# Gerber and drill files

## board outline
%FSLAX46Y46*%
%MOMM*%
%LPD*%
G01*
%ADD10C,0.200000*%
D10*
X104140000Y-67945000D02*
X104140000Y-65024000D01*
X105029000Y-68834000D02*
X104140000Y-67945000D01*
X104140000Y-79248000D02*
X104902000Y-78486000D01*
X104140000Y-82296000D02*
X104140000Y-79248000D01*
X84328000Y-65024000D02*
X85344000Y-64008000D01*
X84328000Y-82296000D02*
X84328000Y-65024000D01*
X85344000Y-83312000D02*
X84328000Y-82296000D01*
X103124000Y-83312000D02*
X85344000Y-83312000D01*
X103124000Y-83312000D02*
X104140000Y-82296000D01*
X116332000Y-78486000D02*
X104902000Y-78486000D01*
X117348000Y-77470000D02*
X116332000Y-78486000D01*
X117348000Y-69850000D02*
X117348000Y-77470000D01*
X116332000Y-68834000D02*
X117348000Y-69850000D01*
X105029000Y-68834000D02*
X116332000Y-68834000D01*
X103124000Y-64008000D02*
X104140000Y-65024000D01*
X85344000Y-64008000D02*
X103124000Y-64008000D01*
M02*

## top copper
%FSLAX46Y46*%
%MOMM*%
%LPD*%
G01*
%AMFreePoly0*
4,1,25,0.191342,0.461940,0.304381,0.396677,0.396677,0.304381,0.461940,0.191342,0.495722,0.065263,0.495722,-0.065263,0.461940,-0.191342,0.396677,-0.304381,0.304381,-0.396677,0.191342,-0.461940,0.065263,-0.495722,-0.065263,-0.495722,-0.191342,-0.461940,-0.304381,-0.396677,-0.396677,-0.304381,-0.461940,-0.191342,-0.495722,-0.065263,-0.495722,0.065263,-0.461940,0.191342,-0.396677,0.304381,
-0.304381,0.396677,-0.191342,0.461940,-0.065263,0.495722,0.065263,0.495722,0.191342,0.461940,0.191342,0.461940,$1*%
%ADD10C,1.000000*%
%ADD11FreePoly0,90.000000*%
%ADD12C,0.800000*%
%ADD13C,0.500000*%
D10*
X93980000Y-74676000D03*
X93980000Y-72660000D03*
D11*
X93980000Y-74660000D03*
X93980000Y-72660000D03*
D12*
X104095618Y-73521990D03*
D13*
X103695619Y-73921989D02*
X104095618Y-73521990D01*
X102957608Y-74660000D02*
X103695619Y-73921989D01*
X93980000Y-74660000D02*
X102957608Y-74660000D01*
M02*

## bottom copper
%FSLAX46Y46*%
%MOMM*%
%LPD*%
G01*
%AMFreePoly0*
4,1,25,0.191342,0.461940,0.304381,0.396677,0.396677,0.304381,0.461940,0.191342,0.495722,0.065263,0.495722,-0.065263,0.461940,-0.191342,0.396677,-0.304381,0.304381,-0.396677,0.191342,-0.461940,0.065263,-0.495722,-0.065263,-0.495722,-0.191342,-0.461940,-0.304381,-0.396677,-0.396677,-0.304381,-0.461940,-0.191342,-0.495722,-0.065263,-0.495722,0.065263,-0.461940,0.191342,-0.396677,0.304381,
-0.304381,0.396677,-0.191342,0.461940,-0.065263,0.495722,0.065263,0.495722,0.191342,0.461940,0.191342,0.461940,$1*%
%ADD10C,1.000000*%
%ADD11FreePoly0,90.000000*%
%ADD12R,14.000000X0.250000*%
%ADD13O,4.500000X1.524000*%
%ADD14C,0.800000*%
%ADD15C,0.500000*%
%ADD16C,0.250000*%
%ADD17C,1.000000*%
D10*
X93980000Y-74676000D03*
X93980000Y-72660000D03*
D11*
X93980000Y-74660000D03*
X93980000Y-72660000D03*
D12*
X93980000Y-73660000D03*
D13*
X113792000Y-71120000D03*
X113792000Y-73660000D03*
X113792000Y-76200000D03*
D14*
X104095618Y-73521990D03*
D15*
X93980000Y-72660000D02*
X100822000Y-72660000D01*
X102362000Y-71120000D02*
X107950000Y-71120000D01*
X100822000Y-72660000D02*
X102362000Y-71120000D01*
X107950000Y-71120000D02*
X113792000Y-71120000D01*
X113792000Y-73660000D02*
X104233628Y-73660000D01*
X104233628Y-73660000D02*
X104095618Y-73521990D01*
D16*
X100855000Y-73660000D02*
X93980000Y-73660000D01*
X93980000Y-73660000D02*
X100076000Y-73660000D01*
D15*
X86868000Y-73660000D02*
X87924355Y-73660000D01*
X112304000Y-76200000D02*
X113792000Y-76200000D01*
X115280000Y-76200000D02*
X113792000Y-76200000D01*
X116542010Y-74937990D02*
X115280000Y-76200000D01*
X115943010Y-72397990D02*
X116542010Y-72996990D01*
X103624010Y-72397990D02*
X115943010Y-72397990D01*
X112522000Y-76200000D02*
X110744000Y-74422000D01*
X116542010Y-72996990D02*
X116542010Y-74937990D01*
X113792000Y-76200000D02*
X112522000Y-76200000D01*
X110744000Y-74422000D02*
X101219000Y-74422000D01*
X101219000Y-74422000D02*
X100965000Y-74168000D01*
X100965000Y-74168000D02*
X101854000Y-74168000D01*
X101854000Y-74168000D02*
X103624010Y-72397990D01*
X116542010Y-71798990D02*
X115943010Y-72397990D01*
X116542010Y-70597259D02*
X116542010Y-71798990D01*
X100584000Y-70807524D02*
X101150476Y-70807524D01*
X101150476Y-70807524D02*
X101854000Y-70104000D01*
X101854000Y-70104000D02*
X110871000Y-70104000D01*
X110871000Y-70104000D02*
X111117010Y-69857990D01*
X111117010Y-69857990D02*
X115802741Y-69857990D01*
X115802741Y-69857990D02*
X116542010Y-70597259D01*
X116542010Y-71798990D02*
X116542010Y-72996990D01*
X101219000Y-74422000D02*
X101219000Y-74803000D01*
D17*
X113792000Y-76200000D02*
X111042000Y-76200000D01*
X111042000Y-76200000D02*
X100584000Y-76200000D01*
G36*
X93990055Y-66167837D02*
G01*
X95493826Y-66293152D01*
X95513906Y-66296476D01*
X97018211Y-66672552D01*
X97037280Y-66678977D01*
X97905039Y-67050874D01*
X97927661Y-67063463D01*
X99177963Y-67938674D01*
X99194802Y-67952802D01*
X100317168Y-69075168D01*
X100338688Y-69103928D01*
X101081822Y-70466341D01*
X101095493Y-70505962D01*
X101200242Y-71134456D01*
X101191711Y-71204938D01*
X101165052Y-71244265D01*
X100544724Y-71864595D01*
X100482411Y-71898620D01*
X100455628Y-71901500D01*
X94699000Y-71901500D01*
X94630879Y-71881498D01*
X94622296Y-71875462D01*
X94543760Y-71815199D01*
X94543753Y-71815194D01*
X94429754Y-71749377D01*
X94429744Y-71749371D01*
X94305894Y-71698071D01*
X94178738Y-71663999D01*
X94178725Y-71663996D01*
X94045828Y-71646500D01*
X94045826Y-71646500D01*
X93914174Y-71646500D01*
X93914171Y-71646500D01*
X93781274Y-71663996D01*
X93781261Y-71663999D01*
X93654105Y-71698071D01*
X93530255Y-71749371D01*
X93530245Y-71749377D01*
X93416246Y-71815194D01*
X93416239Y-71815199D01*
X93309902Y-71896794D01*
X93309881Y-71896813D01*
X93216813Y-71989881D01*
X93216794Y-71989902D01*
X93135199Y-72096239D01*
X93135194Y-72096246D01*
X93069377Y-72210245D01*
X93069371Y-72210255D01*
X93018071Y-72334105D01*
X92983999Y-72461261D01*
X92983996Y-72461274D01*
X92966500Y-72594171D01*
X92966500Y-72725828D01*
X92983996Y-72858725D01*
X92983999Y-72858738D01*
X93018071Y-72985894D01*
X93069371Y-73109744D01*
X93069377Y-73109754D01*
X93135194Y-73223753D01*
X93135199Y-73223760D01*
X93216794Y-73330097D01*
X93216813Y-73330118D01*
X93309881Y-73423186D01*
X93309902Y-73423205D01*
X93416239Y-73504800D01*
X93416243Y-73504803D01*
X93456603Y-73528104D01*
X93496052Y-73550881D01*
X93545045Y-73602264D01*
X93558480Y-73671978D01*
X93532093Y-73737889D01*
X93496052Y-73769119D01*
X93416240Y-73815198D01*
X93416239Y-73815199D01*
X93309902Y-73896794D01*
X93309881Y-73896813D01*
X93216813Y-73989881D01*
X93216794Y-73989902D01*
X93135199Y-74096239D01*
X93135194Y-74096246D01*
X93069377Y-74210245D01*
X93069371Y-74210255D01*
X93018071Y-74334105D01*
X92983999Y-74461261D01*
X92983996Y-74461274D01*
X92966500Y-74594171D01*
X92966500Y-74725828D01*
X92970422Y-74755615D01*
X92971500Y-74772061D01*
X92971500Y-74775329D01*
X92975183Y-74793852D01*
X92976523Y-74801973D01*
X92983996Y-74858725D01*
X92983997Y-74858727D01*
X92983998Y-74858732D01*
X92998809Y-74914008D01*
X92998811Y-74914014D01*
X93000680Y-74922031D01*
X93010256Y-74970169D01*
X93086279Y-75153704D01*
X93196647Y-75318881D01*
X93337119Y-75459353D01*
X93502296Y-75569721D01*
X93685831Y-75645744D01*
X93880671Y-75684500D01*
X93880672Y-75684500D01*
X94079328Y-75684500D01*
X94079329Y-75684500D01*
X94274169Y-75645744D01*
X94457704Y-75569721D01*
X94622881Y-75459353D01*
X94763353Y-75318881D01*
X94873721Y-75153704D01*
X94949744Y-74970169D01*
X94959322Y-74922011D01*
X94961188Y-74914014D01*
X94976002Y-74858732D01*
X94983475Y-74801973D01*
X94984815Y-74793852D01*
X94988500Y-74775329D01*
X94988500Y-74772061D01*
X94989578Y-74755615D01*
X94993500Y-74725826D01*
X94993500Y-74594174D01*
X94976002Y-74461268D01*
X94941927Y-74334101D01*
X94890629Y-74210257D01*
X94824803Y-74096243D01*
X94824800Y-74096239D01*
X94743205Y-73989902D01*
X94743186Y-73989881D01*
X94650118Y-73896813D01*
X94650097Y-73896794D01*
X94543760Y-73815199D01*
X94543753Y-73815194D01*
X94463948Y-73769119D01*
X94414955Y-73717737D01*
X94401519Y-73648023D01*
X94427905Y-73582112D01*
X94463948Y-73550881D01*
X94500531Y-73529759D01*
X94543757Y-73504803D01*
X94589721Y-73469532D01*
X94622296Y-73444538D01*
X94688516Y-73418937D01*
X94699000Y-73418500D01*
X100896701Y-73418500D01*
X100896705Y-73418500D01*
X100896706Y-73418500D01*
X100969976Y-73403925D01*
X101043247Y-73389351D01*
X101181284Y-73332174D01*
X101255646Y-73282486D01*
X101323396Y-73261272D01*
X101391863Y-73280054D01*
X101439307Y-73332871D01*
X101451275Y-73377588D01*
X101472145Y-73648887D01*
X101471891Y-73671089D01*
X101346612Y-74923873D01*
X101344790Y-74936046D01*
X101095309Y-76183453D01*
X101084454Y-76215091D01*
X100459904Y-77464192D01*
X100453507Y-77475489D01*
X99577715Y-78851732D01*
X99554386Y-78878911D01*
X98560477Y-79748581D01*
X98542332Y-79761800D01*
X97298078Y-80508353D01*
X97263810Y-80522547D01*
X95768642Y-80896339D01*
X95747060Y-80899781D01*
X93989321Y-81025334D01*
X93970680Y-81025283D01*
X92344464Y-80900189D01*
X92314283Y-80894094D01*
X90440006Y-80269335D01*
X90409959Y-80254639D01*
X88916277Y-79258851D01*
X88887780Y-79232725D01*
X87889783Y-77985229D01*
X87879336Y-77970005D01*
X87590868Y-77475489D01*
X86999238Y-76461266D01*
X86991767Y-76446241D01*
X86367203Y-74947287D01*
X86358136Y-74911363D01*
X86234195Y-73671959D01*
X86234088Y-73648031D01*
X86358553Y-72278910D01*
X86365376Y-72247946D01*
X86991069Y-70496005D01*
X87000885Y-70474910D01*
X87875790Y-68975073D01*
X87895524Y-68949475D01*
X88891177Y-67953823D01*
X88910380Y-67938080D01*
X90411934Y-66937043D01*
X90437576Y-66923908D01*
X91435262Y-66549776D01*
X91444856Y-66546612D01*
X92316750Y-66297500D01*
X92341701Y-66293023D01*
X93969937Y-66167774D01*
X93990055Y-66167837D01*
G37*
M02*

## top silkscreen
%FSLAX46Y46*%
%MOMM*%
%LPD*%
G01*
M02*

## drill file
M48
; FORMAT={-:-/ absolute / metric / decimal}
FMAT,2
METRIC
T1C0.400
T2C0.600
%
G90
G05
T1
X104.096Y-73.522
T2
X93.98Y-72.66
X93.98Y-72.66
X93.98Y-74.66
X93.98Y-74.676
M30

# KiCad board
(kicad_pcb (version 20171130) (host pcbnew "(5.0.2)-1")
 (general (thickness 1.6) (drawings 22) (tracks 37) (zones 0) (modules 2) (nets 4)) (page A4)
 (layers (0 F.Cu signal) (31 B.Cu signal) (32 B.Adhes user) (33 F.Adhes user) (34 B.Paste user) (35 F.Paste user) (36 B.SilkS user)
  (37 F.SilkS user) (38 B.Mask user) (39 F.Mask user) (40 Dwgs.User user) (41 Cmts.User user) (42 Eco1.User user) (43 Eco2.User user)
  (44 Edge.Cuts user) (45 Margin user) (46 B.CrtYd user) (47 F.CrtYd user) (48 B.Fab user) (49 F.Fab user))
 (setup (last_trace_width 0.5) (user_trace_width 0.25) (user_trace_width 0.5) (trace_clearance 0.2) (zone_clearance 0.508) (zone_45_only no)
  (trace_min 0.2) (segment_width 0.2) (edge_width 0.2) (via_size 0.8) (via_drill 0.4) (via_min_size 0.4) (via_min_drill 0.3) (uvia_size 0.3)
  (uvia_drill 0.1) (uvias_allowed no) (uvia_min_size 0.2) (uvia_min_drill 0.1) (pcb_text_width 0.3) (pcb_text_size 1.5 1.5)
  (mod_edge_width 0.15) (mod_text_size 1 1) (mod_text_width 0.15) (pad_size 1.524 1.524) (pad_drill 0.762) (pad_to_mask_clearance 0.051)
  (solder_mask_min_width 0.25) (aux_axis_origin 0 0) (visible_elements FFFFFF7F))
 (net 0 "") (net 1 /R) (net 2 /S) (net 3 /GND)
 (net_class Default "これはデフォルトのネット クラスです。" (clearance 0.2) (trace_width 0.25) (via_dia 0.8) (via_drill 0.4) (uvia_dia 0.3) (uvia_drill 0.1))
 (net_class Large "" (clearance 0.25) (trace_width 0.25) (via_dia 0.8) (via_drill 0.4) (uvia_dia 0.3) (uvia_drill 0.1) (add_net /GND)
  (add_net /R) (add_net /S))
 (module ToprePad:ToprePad (layer F.Cu) (at 93.98 73.66 90)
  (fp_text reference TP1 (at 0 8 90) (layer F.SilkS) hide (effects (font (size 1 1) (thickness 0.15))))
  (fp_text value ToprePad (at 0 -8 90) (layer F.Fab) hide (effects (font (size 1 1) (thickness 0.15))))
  (pad 2 thru_hole circle (at -1.016 0 90) (size 1 1) (drill 0.6) (layers *.Cu *.Mask) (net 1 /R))
  (pad 1 thru_hole circle (at 1 0 90) (size 1 1) (drill 0.6) (layers *.Cu *.Mask) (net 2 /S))
  (pad 2 thru_hole custom (at -1 0 90) (size 1 1) (drill 0.6) (layers B.Cu) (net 1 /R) (zone_connect 0)
   (options (clearance outline) (anchor circle)) (primitives))
  (pad 1 thru_hole custom (at 1 0 90) (size 1 1) (drill 0.6) (layers B.Cu) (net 2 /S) (zone_connect 0)
   (options (clearance outline) (anchor circle)) (primitives))
  (pad 3 smd rect (at 0 0 90) (size 0.25 14) (layers B.Cu) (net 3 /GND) (zone_connect 2)))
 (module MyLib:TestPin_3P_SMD (layer B.Cu) (at 113.792 71.12)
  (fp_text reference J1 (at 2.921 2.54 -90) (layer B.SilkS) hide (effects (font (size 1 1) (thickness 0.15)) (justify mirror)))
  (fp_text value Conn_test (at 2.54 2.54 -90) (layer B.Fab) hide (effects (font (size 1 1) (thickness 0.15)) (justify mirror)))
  (pad 1 smd oval (at 0 0) (size 4.5 1.524) (layers B.Cu B.Paste B.Mask) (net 2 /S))
  (pad 2 smd oval (at 0 2.54) (size 4.5 1.524) (layers B.Cu B.Paste B.Mask) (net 1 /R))
  (pad 3 smd oval (at 0 5.08) (size 4.5 1.524) (layers B.Cu B.Paste B.Mask) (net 3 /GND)))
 (gr_line (start 104.14 67.945) (end 104.14 65.024) (layer Edge.Cuts) (width 0.2))
 (gr_line (start 105.029 68.834) (end 104.14 67.945) (layer Edge.Cuts) (width 0.2))
 (gr_line (start 104.14 79.248) (end 104.902 78.486) (layer Edge.Cuts) (width 0.2))
 (gr_line (start 104.14 82.296) (end 104.14 79.248) (layer Edge.Cuts) (width 0.2))
 (gr_line (start 84.328 65.024) (end 85.344 64.008) (layer Edge.Cuts) (width 0.2))
 (gr_line (start 84.328 82.296) (end 84.328 65.024) (layer Edge.Cuts) (width 0.2))
 (gr_line (start 85.344 83.312) (end 84.328 82.296) (layer Edge.Cuts) (width 0.2))
 (gr_line (start 103.124 83.312) (end 85.344 83.312) (layer Edge.Cuts) (width 0.2))
 (gr_line (start 103.124 83.312) (end 104.14 82.296) (layer Edge.Cuts) (width 0.2))
 (gr_line (start 116.332 78.486) (end 104.902 78.486) (layer Edge.Cuts) (width 0.2))
 (gr_line (start 117.348 77.47) (end 116.332 78.486) (layer Edge.Cuts) (width 0.2))
 (gr_line (start 117.348 69.85) (end 117.348 77.47) (layer Edge.Cuts) (width 0.2))
 (gr_line (start 116.332 68.834) (end 117.348 69.85) (layer Edge.Cuts) (width 0.2))
 (gr_line (start 105.029 68.834) (end 116.332 68.834) (layer Edge.Cuts) (width 0.2))
 (gr_line (start 103.124 64.008) (end 104.14 65.024) (layer Edge.Cuts) (width 0.2))
 (gr_line (start 85.344 64.008) (end 103.124 64.008) (layer Edge.Cuts) (width 0.2))
 (segment (start 93.98 72.66) (end 100.822 72.66) (width 0.5) (layer B.Cu) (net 2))
 (segment (start 102.362 71.12) (end 107.95 71.12) (width 0.5) (layer B.Cu) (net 2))
 (segment (start 100.822 72.66) (end 102.362 71.12) (width 0.5) (layer B.Cu) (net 2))
 (segment (start 107.95 71.12) (end 113.792 71.12) (width 0.5) (layer B.Cu) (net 2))
 (segment (start 113.792 73.66) (end 104.233628 73.66) (width 0.5) (layer B.Cu) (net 1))
 (segment (start 104.233628 73.66) (end 104.095618 73.52199) (width 0.5) (layer B.Cu) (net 1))
 (segment (start 103.695619 73.921989) (end 104.095618 73.52199) (width 0.5) (layer F.Cu) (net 1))
 (segment (start 102.957608 74.66) (end 103.695619 73.921989) (width 0.5) (layer F.Cu) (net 1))
 (via (at 104.095618 73.52199) (size 0.8) (drill 0.4) (layers F.Cu B.Cu) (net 1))
 (segment (start 93.98 74.66) (end 102.957608 74.66) (width 0.5) (layer F.Cu) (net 1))
 (segment (start 100.855 73.66) (end 93.98 73.66) (width 0.25) (layer B.Cu) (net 3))
 (segment (start 93.98 73.66) (end 100.076 73.66) (width 0.25) (layer B.Cu) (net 3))
 (segment (start 86.868 73.66) (end 87.924355 73.66) (width 0.5) (layer B.Cu) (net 3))
 (segment (start 112.304 76.2) (end 113.792 76.2) (width 0.5) (layer B.Cu) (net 3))
 (segment (start 115.28 76.2) (end 113.792 76.2) (width 0.5) (layer B.Cu) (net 3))
 (segment (start 116.54201 74.93799) (end 115.28 76.2) (width 0.5) (layer B.Cu) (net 3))
 (segment (start 115.94301 72.39799) (end 116.54201 72.99699) (width 0.5) (layer B.Cu) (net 3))
 (segment (start 103.62401 72.39799) (end 115.94301 72.39799) (width 0.5) (layer B.Cu) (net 3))
 (segment (start 112.522 76.2) (end 110.744 74.422) (width 0.5) (layer B.Cu) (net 3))
 (segment (start 116.54201 72.99699) (end 116.54201 74.93799) (width 0.5) (layer B.Cu) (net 3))
 (segment (start 113.792 76.2) (end 112.522 76.2) (width 0.5) (layer B.Cu) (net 3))
 (segment (start 110.744 74.422) (end 101.219 74.422) (width 0.5) (layer B.Cu) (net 3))
 (segment (start 101.219 74.422) (end 100.965 74.168) (width 0.5) (layer B.Cu) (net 3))
 (segment (start 100.965 74.168) (end 101.854 74.168) (width 0.5) (layer B.Cu) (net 3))
 (segment (start 101.854 74.168) (end 103.62401 72.39799) (width 0.5) (layer B.Cu) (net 3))
 (segment (start 116.54201 71.79899) (end 115.94301 72.39799) (width 0.5) (layer B.Cu) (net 3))
 (segment (start 116.54201 70.597259) (end 116.54201 71.79899) (width 0.5) (layer B.Cu) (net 3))
 (segment (start 100.584 70.807524) (end 101.150476 70.807524) (width 0.5) (layer B.Cu) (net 3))
 (segment (start 101.150476 70.807524) (end 101.854 70.104) (width 0.5) (layer B.Cu) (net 3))
 (segment (start 101.854 70.104) (end 110.871 70.104) (width 0.5) (layer B.Cu) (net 3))
 (segment (start 110.871 70.104) (end 111.11701 69.85799) (width 0.5) (layer B.Cu) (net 3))
 (segment (start 111.11701 69.85799) (end 115.802741 69.85799) (width 0.5) (layer B.Cu) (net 3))
 (segment (start 115.802741 69.85799) (end 116.54201 70.597259) (width 0.5) (layer B.Cu) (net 3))
 (segment (start 116.54201 71.79899) (end 116.54201 72.99699) (width 0.5) (layer B.Cu) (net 3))
 (segment (start 101.219 74.422) (end 101.219 74.803) (width 0.5) (layer B.Cu) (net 3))
 (segment (start 113.792 76.2) (end 111.042 76.2) (width 1) (layer B.Cu) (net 3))
 (segment (start 111.042 76.2) (end 100.584 76.2) (width 1) (layer B.Cu) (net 3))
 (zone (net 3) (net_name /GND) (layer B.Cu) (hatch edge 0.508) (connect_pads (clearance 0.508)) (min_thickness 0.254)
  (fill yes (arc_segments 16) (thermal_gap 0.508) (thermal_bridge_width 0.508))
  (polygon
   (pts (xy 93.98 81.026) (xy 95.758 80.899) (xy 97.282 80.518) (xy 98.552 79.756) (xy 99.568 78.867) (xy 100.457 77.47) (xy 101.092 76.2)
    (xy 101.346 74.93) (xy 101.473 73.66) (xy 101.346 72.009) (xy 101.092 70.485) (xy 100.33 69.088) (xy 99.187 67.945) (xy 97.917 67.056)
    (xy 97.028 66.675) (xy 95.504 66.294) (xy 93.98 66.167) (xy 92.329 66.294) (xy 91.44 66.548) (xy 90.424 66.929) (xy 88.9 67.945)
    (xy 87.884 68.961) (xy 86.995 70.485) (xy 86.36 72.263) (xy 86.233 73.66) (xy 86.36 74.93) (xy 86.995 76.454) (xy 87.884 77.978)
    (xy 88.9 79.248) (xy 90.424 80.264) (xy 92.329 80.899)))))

